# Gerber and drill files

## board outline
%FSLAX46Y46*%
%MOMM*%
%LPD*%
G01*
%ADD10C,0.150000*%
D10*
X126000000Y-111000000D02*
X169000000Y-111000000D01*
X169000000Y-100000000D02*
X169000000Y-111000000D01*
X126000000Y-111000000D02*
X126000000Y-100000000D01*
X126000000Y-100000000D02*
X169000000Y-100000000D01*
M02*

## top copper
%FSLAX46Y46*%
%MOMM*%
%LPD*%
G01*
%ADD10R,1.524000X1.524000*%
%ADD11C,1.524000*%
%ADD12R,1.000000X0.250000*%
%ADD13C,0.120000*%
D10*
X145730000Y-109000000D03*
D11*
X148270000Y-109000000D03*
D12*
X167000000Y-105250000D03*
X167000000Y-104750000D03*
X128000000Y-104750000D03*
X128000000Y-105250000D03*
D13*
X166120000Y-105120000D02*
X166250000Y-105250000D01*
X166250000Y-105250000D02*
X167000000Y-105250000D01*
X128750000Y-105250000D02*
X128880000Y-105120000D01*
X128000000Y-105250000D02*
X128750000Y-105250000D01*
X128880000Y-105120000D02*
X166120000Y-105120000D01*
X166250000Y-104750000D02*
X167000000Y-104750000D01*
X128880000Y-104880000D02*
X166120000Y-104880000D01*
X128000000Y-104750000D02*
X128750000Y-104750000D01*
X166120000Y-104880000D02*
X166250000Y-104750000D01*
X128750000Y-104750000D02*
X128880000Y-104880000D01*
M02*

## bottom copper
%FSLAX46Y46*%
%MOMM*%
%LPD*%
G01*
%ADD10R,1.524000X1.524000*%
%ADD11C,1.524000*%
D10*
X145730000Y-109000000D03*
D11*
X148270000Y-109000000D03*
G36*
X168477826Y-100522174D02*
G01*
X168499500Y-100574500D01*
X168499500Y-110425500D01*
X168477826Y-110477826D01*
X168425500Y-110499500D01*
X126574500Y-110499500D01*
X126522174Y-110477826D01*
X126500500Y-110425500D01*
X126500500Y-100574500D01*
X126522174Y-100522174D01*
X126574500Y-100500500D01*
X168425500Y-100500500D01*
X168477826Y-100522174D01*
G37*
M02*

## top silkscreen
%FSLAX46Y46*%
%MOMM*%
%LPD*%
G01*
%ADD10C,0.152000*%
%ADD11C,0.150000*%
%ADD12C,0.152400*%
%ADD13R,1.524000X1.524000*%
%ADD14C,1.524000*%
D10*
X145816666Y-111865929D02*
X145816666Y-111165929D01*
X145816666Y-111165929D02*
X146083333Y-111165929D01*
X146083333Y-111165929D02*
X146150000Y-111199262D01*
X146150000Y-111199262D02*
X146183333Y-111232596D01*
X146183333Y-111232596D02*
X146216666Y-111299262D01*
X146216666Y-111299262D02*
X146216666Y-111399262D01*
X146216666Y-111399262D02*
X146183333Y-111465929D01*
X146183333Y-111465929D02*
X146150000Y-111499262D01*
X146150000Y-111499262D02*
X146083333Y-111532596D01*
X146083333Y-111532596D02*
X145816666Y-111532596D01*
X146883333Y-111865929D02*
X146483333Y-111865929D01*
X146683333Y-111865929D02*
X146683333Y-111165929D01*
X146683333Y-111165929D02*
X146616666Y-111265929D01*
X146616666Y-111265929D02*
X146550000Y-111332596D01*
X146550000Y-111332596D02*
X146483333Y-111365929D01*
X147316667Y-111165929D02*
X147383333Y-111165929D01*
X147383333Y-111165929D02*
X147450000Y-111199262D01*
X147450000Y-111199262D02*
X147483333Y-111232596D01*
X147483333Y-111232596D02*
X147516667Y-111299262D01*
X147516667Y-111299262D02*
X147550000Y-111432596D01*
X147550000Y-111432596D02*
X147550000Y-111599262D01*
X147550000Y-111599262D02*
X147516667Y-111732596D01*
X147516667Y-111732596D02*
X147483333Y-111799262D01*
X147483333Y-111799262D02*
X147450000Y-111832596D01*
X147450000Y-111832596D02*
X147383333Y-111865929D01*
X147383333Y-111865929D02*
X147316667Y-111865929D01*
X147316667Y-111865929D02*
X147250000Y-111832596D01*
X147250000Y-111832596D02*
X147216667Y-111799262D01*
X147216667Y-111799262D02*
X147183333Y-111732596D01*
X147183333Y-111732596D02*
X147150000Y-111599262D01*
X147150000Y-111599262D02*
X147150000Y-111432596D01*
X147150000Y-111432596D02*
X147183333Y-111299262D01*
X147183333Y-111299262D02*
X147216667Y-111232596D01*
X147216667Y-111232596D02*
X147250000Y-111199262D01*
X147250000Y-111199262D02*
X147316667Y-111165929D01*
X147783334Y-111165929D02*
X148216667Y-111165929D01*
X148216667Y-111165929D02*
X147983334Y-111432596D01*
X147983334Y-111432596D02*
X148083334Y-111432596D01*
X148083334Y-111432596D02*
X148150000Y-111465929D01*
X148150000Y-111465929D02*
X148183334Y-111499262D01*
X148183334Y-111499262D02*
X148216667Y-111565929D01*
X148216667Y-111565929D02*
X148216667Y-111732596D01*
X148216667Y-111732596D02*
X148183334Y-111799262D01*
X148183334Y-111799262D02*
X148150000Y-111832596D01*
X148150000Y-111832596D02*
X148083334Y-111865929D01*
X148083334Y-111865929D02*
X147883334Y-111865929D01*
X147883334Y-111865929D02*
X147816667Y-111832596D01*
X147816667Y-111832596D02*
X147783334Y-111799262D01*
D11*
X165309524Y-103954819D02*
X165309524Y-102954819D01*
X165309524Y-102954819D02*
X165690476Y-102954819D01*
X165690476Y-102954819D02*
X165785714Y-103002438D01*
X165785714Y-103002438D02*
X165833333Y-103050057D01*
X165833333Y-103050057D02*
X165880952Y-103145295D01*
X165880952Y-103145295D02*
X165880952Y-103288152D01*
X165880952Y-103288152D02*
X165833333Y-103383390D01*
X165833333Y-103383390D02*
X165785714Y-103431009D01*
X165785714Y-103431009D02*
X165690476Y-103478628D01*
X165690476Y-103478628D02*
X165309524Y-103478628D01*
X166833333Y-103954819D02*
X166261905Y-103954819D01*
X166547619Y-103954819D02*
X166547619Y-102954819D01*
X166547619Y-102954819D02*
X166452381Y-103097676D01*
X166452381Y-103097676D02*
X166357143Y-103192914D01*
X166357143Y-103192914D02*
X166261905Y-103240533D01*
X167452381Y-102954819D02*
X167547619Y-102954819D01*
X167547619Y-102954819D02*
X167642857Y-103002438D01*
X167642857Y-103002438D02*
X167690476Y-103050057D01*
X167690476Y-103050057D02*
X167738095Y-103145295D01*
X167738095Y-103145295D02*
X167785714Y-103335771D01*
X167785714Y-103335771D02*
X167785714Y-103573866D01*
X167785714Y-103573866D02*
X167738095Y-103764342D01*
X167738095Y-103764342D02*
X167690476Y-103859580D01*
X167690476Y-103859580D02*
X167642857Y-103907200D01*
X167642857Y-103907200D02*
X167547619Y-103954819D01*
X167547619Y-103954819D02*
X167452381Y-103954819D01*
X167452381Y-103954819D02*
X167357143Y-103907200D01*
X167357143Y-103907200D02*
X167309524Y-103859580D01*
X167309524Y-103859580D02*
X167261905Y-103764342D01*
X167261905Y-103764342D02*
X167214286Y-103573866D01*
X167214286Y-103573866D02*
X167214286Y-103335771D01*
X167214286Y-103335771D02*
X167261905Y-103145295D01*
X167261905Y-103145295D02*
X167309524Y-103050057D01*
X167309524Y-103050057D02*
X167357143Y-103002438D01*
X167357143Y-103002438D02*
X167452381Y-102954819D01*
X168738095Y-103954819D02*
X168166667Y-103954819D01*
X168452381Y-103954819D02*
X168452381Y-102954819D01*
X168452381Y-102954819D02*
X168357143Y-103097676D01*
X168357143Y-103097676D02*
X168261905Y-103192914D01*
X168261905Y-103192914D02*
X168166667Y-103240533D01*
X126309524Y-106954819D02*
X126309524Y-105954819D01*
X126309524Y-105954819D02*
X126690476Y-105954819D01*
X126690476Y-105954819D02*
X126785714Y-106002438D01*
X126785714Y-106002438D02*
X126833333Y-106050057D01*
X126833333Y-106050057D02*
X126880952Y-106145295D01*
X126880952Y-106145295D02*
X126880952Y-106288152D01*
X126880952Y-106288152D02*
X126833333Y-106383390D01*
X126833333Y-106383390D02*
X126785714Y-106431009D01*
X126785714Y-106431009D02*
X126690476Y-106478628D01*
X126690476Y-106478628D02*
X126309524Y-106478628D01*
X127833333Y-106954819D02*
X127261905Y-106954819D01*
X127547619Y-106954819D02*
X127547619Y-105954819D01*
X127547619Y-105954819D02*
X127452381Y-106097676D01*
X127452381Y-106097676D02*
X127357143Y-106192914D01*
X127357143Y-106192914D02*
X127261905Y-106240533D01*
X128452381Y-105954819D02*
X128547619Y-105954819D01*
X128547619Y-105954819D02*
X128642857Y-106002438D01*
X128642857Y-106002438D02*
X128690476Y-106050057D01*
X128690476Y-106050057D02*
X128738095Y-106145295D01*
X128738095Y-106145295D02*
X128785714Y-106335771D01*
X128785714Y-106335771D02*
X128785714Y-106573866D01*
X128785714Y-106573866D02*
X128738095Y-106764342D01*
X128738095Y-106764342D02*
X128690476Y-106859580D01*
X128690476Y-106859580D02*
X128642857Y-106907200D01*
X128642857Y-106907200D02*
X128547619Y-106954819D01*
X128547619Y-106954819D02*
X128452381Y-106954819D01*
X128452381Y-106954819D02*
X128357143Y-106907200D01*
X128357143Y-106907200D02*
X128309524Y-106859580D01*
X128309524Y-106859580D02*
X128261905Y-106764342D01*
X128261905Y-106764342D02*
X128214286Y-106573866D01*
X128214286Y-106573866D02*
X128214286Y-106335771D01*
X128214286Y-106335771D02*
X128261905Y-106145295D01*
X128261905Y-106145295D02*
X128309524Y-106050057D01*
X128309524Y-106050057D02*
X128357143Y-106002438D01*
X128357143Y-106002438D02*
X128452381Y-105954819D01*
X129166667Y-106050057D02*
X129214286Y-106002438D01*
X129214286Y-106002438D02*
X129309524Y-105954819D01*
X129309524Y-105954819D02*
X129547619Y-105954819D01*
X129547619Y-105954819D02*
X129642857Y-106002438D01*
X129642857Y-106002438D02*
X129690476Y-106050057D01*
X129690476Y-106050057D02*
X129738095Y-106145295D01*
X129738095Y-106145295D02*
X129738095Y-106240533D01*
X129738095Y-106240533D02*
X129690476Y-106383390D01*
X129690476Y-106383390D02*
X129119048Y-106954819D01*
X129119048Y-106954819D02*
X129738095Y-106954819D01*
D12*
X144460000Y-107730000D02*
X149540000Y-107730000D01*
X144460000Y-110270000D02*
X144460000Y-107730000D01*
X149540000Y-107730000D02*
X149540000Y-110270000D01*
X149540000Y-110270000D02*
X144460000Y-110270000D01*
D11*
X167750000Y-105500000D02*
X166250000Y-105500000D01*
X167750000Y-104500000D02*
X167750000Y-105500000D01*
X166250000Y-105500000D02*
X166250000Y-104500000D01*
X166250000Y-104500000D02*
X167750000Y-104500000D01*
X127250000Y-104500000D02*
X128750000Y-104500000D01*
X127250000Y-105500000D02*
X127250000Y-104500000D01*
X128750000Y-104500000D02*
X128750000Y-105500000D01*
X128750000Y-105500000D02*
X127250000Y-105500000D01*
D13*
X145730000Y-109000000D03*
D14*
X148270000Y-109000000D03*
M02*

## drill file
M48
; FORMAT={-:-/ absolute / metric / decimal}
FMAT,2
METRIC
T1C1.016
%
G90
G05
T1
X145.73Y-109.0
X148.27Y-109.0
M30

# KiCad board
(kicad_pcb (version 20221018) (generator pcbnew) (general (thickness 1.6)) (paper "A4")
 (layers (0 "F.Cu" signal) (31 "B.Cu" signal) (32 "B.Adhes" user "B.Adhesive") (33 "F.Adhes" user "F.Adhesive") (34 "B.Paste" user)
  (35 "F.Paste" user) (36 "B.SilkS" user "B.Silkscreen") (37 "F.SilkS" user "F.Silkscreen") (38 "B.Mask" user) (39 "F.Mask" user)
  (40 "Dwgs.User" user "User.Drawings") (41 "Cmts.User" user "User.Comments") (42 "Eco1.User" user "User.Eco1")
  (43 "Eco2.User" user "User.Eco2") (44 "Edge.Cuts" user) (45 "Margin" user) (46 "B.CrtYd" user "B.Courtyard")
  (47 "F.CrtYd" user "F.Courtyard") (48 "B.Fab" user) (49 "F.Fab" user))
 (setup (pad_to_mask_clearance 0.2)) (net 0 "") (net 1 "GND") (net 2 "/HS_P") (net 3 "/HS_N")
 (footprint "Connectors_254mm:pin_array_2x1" (layer "F.Cu") (at 147 109)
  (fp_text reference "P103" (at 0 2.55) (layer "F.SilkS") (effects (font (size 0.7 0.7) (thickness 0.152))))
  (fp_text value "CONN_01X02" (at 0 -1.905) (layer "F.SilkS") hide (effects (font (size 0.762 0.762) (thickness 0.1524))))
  (fp_line (start -2.54 -1.27) (end 2.54 -1.27) (stroke (width 0.1524) (type solid)) (layer "F.SilkS"))
  (fp_line (start -2.54 1.27) (end -2.54 -1.27) (stroke (width 0.1524) (type solid)) (layer "F.SilkS"))
  (fp_line (start 2.54 -1.27) (end 2.54 1.27) (stroke (width 0.1524) (type solid)) (layer "F.SilkS"))
  (fp_line (start 2.54 1.27) (end -2.54 1.27) (stroke (width 0.1524) (type solid)) (layer "F.SilkS"))
  (pad "1" thru_hole rect (at -1.27 0) (size 1.524 1.524) (drill 1.016) (layers "*.Cu" "*.Mask" "F.SilkS") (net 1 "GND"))
  (pad "2" thru_hole circle (at 1.27 0) (size 1.524 1.524) (drill 1.016) (layers "*.Cu" "*.Mask" "F.SilkS") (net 1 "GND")))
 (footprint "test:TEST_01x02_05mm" (layer "F.Cu") (at 167 105 180)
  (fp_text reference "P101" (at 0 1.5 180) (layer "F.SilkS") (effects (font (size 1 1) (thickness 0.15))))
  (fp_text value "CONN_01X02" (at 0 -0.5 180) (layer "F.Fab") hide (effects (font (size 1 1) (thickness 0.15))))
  (fp_line (start -0.75 -0.5) (end 0.75 -0.5) (stroke (width 0.15) (type solid)) (layer "F.SilkS"))
  (fp_line (start -0.75 0.5) (end -0.75 -0.5) (stroke (width 0.15) (type solid)) (layer "F.SilkS"))
  (fp_line (start 0.75 -0.5) (end 0.75 0.5) (stroke (width 0.15) (type solid)) (layer "F.SilkS"))
  (fp_line (start 0.75 0.5) (end -0.75 0.5) (stroke (width 0.15) (type solid)) (layer "F.SilkS"))
  (pad "1" smd rect (at 0 -0.25 180) (size 1 0.25) (layers "F.Cu" "F.Paste" "F.Mask") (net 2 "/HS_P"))
  (pad "2" smd rect (at 0 0.25 180) (size 1 0.25) (layers "F.Cu" "F.Paste" "F.Mask") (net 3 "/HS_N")))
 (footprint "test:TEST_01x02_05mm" (layer "F.Cu") (at 128 105)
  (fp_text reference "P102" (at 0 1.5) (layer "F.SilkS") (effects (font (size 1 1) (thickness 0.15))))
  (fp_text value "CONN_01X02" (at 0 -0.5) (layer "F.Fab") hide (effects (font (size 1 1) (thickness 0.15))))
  (fp_line (start -0.75 -0.5) (end 0.75 -0.5) (stroke (width 0.15) (type solid)) (layer "F.SilkS"))
  (fp_line (start -0.75 0.5) (end -0.75 -0.5) (stroke (width 0.15) (type solid)) (layer "F.SilkS"))
  (fp_line (start 0.75 -0.5) (end 0.75 0.5) (stroke (width 0.15) (type solid)) (layer "F.SilkS"))
  (fp_line (start 0.75 0.5) (end -0.75 0.5) (stroke (width 0.15) (type solid)) (layer "F.SilkS"))
  (pad "1" smd rect (at 0 -0.25) (size 1 0.25) (layers "F.Cu" "F.Paste" "F.Mask") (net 3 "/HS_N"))
  (pad "2" smd rect (at 0 0.25) (size 1 0.25) (layers "F.Cu" "F.Paste" "F.Mask") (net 2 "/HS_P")))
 (gr_line (start 126 111) (end 169 111) (stroke (width 0.15) (type solid)) (layer "Edge.Cuts"))
 (gr_line (start 169 100) (end 169 111) (stroke (width 0.15) (type solid)) (layer "Edge.Cuts"))
 (gr_line (start 126 111) (end 126 100) (stroke (width 0.15) (type solid)) (layer "Edge.Cuts"))
 (gr_line (start 126 100) (end 169 100) (stroke (width 0.15) (type solid)) (layer "Edge.Cuts"))
 (segment (start 166.12 105.12) (end 166.25 105.25) (width 0.12) (layer "F.Cu") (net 2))
 (segment (start 166.25 105.25) (end 167 105.25) (width 0.12) (layer "F.Cu") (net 2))
 (segment (start 128.75 105.25) (end 128.88 105.12) (width 0.12) (layer "F.Cu") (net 2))
 (segment (start 128 105.25) (end 128.75 105.25) (width 0.12) (layer "F.Cu") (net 2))
 (segment (start 128.88 105.12) (end 166.12 105.12) (width 0.12) (layer "F.Cu") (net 2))
 (segment (start 166.25 104.75) (end 167 104.75) (width 0.12) (layer "F.Cu") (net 3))
 (segment (start 128.88 104.88) (end 166.12 104.88) (width 0.12) (layer "F.Cu") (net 3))
 (segment (start 128 104.75) (end 128.75 104.75) (width 0.12) (layer "F.Cu") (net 3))
 (segment (start 166.12 104.88) (end 166.25 104.75) (width 0.12) (layer "F.Cu") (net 3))
 (segment (start 128.75 104.75) (end 128.88 104.88) (width 0.12) (layer "F.Cu") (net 3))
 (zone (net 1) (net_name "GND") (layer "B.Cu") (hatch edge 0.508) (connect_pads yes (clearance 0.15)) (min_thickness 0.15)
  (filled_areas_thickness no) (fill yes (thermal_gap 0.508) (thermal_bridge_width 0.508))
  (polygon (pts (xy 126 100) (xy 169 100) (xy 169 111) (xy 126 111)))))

